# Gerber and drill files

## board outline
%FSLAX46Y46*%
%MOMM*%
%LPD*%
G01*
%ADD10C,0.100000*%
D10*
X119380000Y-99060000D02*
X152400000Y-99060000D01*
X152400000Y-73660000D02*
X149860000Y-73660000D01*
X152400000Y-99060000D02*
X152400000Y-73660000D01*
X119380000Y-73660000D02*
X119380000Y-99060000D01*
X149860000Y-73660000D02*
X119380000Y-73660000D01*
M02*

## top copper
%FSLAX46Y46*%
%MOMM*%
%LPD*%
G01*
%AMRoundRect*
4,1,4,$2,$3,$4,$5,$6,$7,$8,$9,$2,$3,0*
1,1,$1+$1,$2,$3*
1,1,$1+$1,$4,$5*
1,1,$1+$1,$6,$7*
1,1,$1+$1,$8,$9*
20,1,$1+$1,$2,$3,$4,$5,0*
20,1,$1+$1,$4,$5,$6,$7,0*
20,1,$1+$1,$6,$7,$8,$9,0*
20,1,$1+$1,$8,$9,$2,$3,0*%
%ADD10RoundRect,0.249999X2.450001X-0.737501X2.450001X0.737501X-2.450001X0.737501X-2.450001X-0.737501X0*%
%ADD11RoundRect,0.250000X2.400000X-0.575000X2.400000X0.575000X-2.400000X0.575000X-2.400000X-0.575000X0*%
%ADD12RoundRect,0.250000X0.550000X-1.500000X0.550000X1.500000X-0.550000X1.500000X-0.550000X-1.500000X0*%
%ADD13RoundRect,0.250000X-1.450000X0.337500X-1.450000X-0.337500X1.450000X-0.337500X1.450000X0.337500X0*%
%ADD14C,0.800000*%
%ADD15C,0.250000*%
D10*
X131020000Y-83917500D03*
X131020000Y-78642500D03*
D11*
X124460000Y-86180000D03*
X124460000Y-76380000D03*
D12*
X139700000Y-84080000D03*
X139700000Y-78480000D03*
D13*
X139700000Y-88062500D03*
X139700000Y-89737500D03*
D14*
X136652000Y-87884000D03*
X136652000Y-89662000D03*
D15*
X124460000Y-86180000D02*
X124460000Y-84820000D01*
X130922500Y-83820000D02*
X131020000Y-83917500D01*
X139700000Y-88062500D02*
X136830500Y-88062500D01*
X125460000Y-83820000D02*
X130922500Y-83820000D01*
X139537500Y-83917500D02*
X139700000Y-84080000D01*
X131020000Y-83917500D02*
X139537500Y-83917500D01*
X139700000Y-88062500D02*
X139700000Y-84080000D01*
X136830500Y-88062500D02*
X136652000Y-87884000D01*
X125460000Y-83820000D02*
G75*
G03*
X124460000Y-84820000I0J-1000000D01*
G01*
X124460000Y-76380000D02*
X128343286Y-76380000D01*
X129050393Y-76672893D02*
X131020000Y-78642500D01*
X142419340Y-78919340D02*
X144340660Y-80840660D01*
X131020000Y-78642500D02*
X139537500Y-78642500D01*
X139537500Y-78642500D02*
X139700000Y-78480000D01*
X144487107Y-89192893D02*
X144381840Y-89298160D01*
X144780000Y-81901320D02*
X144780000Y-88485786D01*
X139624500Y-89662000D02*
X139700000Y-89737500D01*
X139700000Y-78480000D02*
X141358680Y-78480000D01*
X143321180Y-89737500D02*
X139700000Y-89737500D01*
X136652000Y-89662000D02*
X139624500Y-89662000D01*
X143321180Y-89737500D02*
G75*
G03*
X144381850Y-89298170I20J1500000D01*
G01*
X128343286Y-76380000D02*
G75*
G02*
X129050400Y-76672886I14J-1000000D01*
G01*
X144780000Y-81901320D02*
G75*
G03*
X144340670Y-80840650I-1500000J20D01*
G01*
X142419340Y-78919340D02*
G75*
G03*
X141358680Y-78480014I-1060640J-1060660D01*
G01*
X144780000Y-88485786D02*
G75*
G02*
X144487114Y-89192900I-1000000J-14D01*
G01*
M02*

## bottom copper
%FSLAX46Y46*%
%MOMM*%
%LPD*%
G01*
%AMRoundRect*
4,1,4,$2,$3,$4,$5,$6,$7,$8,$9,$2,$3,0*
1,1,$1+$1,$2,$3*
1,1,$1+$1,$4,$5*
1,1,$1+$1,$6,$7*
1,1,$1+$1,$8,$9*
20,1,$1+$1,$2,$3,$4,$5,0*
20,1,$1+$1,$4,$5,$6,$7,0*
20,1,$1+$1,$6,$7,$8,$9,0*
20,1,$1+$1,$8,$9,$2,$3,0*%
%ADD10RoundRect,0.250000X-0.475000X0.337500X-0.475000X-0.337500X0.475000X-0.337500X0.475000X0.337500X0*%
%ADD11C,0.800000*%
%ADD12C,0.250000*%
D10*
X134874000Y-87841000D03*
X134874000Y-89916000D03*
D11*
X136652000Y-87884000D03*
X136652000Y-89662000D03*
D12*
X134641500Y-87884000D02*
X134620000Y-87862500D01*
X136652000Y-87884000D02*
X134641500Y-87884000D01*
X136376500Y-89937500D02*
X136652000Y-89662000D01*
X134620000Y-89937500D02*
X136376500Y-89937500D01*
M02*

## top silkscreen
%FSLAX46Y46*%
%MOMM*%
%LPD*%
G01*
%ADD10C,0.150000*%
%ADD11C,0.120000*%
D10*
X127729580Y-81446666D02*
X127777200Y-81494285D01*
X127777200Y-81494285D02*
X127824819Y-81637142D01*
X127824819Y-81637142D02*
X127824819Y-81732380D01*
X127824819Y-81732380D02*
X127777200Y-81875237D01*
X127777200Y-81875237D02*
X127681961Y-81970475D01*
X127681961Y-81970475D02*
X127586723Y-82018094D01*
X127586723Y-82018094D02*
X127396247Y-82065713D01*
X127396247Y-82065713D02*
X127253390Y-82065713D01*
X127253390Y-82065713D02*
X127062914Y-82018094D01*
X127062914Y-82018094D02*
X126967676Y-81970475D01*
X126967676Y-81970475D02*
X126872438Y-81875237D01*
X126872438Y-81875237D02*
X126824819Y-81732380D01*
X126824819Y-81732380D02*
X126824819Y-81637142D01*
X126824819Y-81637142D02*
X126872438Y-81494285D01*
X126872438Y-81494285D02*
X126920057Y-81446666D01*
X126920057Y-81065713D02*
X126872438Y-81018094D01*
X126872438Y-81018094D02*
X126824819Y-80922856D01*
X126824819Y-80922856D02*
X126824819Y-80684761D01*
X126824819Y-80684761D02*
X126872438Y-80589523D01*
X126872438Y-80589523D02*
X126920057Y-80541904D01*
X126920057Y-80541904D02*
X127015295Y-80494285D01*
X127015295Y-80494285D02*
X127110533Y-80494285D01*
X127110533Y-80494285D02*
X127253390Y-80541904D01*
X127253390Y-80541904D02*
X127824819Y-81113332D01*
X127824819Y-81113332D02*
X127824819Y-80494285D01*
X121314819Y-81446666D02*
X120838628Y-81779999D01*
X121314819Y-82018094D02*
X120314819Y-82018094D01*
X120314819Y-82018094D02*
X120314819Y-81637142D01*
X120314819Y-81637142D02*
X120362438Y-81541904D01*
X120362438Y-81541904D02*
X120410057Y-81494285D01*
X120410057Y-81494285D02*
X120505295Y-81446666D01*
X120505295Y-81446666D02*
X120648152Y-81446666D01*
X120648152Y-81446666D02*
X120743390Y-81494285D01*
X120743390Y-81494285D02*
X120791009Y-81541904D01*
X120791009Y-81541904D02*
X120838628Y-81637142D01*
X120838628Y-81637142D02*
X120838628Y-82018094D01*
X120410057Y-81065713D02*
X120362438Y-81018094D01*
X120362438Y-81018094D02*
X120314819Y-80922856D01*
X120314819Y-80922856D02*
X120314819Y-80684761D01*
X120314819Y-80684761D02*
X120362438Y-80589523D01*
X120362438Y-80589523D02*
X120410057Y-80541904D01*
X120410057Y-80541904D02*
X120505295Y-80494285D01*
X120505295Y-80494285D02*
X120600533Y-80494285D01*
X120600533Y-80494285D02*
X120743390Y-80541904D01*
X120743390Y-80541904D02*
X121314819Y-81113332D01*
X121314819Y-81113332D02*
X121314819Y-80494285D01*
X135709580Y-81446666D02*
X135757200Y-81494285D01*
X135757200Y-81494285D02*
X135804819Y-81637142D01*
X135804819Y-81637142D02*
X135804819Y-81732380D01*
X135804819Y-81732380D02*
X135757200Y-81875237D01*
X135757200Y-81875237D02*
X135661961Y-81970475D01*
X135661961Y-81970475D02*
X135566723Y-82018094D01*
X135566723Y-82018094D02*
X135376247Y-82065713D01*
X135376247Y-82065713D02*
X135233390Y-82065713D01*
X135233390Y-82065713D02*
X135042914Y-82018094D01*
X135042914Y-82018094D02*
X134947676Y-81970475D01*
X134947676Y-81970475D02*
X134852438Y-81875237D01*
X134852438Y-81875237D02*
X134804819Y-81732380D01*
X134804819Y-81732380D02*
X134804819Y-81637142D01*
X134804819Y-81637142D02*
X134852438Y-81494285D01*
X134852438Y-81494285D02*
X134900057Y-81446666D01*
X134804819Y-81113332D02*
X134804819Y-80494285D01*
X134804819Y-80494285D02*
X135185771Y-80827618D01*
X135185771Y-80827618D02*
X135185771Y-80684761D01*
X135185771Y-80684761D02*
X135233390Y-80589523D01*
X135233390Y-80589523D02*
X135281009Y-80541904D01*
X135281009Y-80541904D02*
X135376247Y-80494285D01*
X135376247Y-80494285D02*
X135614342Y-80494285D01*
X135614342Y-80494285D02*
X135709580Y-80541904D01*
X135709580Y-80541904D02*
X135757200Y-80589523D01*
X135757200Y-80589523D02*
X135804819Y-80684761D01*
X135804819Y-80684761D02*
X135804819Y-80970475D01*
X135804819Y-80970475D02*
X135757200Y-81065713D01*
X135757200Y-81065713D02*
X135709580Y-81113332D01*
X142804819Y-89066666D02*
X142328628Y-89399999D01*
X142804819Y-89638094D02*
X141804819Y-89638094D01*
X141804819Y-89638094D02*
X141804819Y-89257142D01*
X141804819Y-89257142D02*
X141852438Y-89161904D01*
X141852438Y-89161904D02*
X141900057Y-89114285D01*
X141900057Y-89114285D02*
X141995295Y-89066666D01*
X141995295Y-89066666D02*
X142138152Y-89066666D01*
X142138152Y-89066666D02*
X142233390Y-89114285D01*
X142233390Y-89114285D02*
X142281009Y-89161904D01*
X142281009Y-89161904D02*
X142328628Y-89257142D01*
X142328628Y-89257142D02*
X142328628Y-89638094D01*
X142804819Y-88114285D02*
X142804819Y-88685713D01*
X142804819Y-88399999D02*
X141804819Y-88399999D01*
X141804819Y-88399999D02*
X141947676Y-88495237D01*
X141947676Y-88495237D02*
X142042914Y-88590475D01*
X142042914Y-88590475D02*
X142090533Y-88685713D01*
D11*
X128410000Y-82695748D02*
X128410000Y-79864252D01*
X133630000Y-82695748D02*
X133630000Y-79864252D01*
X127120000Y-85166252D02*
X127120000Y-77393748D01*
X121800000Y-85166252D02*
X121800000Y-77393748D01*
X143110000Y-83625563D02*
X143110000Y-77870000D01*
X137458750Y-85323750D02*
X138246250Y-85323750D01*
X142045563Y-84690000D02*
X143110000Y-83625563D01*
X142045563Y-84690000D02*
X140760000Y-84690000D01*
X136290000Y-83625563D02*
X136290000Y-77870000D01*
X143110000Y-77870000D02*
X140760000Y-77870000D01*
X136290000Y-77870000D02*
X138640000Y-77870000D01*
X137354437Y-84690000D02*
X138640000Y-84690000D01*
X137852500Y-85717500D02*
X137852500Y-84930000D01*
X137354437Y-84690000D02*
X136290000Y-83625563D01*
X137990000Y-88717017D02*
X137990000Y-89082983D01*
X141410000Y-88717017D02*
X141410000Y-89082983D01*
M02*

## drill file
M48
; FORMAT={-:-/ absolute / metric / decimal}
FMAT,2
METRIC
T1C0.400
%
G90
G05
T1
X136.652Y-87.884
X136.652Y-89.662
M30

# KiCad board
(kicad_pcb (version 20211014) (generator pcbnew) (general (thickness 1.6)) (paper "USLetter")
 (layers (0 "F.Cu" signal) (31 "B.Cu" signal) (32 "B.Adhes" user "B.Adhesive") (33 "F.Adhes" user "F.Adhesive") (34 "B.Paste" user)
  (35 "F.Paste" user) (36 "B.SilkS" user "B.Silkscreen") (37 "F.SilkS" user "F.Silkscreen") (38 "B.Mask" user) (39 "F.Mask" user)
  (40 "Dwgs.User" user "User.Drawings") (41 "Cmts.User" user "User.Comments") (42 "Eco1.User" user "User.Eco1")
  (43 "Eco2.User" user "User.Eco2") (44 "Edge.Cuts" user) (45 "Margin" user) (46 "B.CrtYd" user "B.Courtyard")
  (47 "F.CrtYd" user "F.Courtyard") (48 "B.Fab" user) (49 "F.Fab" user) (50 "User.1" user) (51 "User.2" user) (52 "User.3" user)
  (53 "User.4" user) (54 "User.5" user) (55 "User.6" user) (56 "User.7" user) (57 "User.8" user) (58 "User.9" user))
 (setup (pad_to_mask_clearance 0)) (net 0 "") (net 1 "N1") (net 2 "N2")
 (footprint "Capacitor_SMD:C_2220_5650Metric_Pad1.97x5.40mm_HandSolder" (layer "F.Cu") (at 131.02 81.28 90)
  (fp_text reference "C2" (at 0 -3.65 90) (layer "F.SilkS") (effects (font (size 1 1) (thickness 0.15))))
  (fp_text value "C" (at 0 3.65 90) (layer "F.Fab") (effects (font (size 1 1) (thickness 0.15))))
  (fp_line (start -1.415748 -2.61) (end 1.415748 -2.61) (layer "F.SilkS") (width 0.12))
  (fp_line (start -1.415748 2.61) (end 1.415748 2.61) (layer "F.SilkS") (width 0.12))
  (pad "1" smd roundrect (at -2.6375 0 90) (size 1.975 5.4) (layers "F.Cu" "F.Paste" "F.Mask") (roundrect_rratio 0.126582) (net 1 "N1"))
  (pad "2" smd roundrect (at 2.6375 0 90) (size 1.975 5.4) (layers "F.Cu" "F.Paste" "F.Mask") (roundrect_rratio 0.126582) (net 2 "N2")))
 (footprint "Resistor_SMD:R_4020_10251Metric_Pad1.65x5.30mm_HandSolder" (layer "F.Cu") (at 124.46 81.28 90)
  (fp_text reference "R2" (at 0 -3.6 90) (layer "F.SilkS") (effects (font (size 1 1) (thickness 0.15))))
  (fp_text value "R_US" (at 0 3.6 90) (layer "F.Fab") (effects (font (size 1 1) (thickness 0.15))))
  (fp_line (start -3.886252 2.66) (end 3.886252 2.66) (layer "F.SilkS") (width 0.12))
  (fp_line (start -3.886252 -2.66) (end 3.886252 -2.66) (layer "F.SilkS") (width 0.12))
  (pad "1" smd roundrect (at -4.9 0 90) (size 1.65 5.3) (layers "F.Cu" "F.Paste" "F.Mask") (roundrect_rratio 0.151515) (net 1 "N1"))
  (pad "2" smd roundrect (at 4.9 0 90) (size 1.65 5.3) (layers "F.Cu" "F.Paste" "F.Mask") (roundrect_rratio 0.151515) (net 2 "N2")))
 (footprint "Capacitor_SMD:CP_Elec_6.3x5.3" (layer "F.Cu") (at 139.7 81.28 90)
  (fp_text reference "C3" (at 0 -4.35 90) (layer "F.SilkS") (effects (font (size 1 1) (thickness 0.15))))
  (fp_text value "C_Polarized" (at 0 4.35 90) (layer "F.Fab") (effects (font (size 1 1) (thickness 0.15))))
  (fp_line (start -2.345563 3.41) (end 3.41 3.41) (layer "F.SilkS") (width 0.12))
  (fp_line (start -4.04375 -2.24125) (end -4.04375 -1.45375) (layer "F.SilkS") (width 0.12))
  (fp_line (start -3.41 2.345563) (end -2.345563 3.41) (layer "F.SilkS") (width 0.12))
  (fp_line (start -3.41 2.345563) (end -3.41 1.06) (layer "F.SilkS") (width 0.12))
  (fp_line (start -2.345563 -3.41) (end 3.41 -3.41) (layer "F.SilkS") (width 0.12))
  (fp_line (start 3.41 3.41) (end 3.41 1.06) (layer "F.SilkS") (width 0.12))
  (fp_line (start 3.41 -3.41) (end 3.41 -1.06) (layer "F.SilkS") (width 0.12))
  (fp_line (start -3.41 -2.345563) (end -3.41 -1.06) (layer "F.SilkS") (width 0.12))
  (fp_line (start -4.4375 -1.8475) (end -3.65 -1.8475) (layer "F.SilkS") (width 0.12))
  (fp_line (start -3.41 -2.345563) (end -2.345563 -3.41) (layer "F.SilkS") (width 0.12))
  (pad "1" smd roundrect (at -2.8 0 90) (size 3.5 1.6) (layers "F.Cu" "F.Paste" "F.Mask") (roundrect_rratio 0.15625) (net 1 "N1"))
  (pad "2" smd roundrect (at 2.8 0 90) (size 3.5 1.6) (layers "F.Cu" "F.Paste" "F.Mask") (roundrect_rratio 0.15625) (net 2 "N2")))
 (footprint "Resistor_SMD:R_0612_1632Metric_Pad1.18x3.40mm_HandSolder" (layer "F.Cu") (at 139.7 88.9 -90)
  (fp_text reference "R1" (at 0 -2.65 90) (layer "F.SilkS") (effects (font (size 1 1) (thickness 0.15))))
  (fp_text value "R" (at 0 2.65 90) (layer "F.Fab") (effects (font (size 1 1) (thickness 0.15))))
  (fp_line (start -0.182983 1.71) (end 0.182983 1.71) (layer "F.SilkS") (width 0.12))
  (fp_line (start -0.182983 -1.71) (end 0.182983 -1.71) (layer "F.SilkS") (width 0.12))
  (pad "1" smd roundrect (at -0.8375 0 270) (size 1.175 3.4) (layers "F.Cu" "F.Paste" "F.Mask") (roundrect_rratio 0.212766) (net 1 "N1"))
  (pad "2" smd roundrect (at 0.8375 0 270) (size 1.175 3.4) (layers "F.Cu" "F.Paste" "F.Mask") (roundrect_rratio 0.212766) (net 2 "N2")))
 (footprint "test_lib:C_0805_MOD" (layer "B.Cu") (at 134.874 88.8785 -90)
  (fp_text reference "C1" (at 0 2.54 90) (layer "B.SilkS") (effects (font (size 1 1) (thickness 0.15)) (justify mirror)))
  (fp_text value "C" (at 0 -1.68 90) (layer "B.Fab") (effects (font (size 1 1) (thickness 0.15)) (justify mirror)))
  (pad "1" smd roundrect (at -1.0375 0 270) (size 1.175 1.45) (layers "B.Cu" "B.Paste" "B.Mask") (roundrect_rratio 0.212766) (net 1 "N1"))
  (pad "2" smd roundrect (at 1.0375 0 270) (size 1.175 1.45) (layers "B.Cu" "B.Paste" "B.Mask") (roundrect_rratio 0.212766) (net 2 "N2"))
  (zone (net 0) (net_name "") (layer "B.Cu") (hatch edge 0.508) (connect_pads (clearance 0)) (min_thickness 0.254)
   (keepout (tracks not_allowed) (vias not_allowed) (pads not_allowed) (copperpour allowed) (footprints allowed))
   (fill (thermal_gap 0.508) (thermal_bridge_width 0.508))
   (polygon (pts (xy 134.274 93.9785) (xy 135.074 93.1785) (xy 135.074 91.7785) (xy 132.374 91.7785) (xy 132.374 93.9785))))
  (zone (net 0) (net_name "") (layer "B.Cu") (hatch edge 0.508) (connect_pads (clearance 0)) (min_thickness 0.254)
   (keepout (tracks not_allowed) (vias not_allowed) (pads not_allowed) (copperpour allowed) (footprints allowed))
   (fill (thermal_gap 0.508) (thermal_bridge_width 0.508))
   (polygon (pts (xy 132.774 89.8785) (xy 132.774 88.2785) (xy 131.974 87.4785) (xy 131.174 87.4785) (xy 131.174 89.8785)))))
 (gr_line (start 119.38 99.06) (end 152.4 99.06) (layer "Edge.Cuts") (width 0.1))
 (gr_line (start 152.4 73.66) (end 149.86 73.66) (layer "Edge.Cuts") (width 0.1))
 (gr_line (start 152.4 99.06) (end 152.4 73.66) (layer "Edge.Cuts") (width 0.1))
 (gr_line (start 119.38 73.66) (end 119.38 99.06) (layer "Edge.Cuts") (width 0.1))
 (gr_line (start 149.86 73.66) (end 119.38 73.66) (layer "Edge.Cuts") (width 0.1))
 (segment (start 124.46 86.18) (end 124.46 84.82) (width 0.25) (layer "F.Cu") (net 1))
 (segment (start 130.9225 83.82) (end 131.02 83.9175) (width 0.25) (layer "F.Cu") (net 1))
 (segment (start 139.7 88.0625) (end 136.8305 88.0625) (width 0.25) (layer "F.Cu") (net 1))
 (segment (start 125.46 83.82) (end 130.9225 83.82) (width 0.25) (layer "F.Cu") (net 1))
 (segment (start 139.5375 83.9175) (end 139.7 84.08) (width 0.25) (layer "F.Cu") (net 1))
 (segment (start 131.02 83.9175) (end 139.5375 83.9175) (width 0.25) (layer "F.Cu") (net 1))
 (segment (start 139.7 88.0625) (end 139.7 84.08) (width 0.25) (layer "F.Cu") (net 1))
 (segment (start 136.8305 88.0625) (end 136.652 87.884) (width 0.25) (layer "F.Cu") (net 1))
 (via (at 136.652 87.884) (size 0.8) (drill 0.4) (layers "F.Cu" "B.Cu") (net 1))
 (arc (start 125.46 83.82) (mid 124.752893 84.112893) (end 124.46 84.82) (width 0.25) (layer "F.Cu") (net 1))
 (segment (start 134.6415 87.884) (end 134.62 87.8625) (width 0.25) (layer "B.Cu") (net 1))
 (segment (start 136.652 87.884) (end 134.6415 87.884) (width 0.25) (layer "B.Cu") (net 1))
 (segment (start 124.46 76.38) (end 128.343286 76.38) (width 0.25) (layer "F.Cu") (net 2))
 (segment (start 129.050393 76.672893) (end 131.02 78.6425) (width 0.25) (layer "F.Cu") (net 2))
 (segment (start 142.41934 78.91934) (end 144.34066 80.84066) (width 0.25) (layer "F.Cu") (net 2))
 (segment (start 131.02 78.6425) (end 139.5375 78.6425) (width 0.25) (layer "F.Cu") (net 2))
 (segment (start 139.5375 78.6425) (end 139.7 78.48) (width 0.25) (layer "F.Cu") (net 2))
 (segment (start 144.487107 89.192893) (end 144.38184 89.29816) (width 0.25) (layer "F.Cu") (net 2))
 (segment (start 144.78 81.90132) (end 144.78 88.485786) (width 0.25) (layer "F.Cu") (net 2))
 (segment (start 139.6245 89.662) (end 139.7 89.7375) (width 0.25) (layer "F.Cu") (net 2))
 (segment (start 139.7 78.48) (end 141.35868 78.48) (width 0.25) (layer "F.Cu") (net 2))
 (segment (start 143.32118 89.7375) (end 139.7 89.7375) (width 0.25) (layer "F.Cu") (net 2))
 (segment (start 136.652 89.662) (end 139.6245 89.662) (width 0.25) (layer "F.Cu") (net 2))
 (via (at 136.652 89.662) (size 0.8) (drill 0.4) (layers "F.Cu" "B.Cu") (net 2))
 (arc (start 143.32118 89.7375) (mid 143.895205 89.623319) (end 144.38184 89.29816) (width 0.25) (layer "F.Cu") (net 2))
 (arc (start 128.343286 76.38) (mid 128.725969 76.45612) (end 129.050393 76.672893) (width 0.25) (layer "F.Cu") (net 2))
 (arc (start 144.78 81.90132) (mid 144.665819 81.327295) (end 144.34066 80.84066) (width 0.25) (layer "F.Cu") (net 2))
 (arc (start 142.41934 78.91934) (mid 141.932705 78.594181) (end 141.35868 78.48) (width 0.25) (layer "F.Cu") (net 2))
 (arc (start 144.78 88.485786) (mid 144.70388 88.868469) (end 144.487107 89.192893) (width 0.25) (layer "F.Cu") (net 2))
 (segment (start 136.3765 89.9375) (end 136.652 89.662) (width 0.25) (layer "B.Cu") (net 2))
 (segment (start 134.62 89.9375) (end 136.3765 89.9375) (width 0.25) (layer "B.Cu") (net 2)))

